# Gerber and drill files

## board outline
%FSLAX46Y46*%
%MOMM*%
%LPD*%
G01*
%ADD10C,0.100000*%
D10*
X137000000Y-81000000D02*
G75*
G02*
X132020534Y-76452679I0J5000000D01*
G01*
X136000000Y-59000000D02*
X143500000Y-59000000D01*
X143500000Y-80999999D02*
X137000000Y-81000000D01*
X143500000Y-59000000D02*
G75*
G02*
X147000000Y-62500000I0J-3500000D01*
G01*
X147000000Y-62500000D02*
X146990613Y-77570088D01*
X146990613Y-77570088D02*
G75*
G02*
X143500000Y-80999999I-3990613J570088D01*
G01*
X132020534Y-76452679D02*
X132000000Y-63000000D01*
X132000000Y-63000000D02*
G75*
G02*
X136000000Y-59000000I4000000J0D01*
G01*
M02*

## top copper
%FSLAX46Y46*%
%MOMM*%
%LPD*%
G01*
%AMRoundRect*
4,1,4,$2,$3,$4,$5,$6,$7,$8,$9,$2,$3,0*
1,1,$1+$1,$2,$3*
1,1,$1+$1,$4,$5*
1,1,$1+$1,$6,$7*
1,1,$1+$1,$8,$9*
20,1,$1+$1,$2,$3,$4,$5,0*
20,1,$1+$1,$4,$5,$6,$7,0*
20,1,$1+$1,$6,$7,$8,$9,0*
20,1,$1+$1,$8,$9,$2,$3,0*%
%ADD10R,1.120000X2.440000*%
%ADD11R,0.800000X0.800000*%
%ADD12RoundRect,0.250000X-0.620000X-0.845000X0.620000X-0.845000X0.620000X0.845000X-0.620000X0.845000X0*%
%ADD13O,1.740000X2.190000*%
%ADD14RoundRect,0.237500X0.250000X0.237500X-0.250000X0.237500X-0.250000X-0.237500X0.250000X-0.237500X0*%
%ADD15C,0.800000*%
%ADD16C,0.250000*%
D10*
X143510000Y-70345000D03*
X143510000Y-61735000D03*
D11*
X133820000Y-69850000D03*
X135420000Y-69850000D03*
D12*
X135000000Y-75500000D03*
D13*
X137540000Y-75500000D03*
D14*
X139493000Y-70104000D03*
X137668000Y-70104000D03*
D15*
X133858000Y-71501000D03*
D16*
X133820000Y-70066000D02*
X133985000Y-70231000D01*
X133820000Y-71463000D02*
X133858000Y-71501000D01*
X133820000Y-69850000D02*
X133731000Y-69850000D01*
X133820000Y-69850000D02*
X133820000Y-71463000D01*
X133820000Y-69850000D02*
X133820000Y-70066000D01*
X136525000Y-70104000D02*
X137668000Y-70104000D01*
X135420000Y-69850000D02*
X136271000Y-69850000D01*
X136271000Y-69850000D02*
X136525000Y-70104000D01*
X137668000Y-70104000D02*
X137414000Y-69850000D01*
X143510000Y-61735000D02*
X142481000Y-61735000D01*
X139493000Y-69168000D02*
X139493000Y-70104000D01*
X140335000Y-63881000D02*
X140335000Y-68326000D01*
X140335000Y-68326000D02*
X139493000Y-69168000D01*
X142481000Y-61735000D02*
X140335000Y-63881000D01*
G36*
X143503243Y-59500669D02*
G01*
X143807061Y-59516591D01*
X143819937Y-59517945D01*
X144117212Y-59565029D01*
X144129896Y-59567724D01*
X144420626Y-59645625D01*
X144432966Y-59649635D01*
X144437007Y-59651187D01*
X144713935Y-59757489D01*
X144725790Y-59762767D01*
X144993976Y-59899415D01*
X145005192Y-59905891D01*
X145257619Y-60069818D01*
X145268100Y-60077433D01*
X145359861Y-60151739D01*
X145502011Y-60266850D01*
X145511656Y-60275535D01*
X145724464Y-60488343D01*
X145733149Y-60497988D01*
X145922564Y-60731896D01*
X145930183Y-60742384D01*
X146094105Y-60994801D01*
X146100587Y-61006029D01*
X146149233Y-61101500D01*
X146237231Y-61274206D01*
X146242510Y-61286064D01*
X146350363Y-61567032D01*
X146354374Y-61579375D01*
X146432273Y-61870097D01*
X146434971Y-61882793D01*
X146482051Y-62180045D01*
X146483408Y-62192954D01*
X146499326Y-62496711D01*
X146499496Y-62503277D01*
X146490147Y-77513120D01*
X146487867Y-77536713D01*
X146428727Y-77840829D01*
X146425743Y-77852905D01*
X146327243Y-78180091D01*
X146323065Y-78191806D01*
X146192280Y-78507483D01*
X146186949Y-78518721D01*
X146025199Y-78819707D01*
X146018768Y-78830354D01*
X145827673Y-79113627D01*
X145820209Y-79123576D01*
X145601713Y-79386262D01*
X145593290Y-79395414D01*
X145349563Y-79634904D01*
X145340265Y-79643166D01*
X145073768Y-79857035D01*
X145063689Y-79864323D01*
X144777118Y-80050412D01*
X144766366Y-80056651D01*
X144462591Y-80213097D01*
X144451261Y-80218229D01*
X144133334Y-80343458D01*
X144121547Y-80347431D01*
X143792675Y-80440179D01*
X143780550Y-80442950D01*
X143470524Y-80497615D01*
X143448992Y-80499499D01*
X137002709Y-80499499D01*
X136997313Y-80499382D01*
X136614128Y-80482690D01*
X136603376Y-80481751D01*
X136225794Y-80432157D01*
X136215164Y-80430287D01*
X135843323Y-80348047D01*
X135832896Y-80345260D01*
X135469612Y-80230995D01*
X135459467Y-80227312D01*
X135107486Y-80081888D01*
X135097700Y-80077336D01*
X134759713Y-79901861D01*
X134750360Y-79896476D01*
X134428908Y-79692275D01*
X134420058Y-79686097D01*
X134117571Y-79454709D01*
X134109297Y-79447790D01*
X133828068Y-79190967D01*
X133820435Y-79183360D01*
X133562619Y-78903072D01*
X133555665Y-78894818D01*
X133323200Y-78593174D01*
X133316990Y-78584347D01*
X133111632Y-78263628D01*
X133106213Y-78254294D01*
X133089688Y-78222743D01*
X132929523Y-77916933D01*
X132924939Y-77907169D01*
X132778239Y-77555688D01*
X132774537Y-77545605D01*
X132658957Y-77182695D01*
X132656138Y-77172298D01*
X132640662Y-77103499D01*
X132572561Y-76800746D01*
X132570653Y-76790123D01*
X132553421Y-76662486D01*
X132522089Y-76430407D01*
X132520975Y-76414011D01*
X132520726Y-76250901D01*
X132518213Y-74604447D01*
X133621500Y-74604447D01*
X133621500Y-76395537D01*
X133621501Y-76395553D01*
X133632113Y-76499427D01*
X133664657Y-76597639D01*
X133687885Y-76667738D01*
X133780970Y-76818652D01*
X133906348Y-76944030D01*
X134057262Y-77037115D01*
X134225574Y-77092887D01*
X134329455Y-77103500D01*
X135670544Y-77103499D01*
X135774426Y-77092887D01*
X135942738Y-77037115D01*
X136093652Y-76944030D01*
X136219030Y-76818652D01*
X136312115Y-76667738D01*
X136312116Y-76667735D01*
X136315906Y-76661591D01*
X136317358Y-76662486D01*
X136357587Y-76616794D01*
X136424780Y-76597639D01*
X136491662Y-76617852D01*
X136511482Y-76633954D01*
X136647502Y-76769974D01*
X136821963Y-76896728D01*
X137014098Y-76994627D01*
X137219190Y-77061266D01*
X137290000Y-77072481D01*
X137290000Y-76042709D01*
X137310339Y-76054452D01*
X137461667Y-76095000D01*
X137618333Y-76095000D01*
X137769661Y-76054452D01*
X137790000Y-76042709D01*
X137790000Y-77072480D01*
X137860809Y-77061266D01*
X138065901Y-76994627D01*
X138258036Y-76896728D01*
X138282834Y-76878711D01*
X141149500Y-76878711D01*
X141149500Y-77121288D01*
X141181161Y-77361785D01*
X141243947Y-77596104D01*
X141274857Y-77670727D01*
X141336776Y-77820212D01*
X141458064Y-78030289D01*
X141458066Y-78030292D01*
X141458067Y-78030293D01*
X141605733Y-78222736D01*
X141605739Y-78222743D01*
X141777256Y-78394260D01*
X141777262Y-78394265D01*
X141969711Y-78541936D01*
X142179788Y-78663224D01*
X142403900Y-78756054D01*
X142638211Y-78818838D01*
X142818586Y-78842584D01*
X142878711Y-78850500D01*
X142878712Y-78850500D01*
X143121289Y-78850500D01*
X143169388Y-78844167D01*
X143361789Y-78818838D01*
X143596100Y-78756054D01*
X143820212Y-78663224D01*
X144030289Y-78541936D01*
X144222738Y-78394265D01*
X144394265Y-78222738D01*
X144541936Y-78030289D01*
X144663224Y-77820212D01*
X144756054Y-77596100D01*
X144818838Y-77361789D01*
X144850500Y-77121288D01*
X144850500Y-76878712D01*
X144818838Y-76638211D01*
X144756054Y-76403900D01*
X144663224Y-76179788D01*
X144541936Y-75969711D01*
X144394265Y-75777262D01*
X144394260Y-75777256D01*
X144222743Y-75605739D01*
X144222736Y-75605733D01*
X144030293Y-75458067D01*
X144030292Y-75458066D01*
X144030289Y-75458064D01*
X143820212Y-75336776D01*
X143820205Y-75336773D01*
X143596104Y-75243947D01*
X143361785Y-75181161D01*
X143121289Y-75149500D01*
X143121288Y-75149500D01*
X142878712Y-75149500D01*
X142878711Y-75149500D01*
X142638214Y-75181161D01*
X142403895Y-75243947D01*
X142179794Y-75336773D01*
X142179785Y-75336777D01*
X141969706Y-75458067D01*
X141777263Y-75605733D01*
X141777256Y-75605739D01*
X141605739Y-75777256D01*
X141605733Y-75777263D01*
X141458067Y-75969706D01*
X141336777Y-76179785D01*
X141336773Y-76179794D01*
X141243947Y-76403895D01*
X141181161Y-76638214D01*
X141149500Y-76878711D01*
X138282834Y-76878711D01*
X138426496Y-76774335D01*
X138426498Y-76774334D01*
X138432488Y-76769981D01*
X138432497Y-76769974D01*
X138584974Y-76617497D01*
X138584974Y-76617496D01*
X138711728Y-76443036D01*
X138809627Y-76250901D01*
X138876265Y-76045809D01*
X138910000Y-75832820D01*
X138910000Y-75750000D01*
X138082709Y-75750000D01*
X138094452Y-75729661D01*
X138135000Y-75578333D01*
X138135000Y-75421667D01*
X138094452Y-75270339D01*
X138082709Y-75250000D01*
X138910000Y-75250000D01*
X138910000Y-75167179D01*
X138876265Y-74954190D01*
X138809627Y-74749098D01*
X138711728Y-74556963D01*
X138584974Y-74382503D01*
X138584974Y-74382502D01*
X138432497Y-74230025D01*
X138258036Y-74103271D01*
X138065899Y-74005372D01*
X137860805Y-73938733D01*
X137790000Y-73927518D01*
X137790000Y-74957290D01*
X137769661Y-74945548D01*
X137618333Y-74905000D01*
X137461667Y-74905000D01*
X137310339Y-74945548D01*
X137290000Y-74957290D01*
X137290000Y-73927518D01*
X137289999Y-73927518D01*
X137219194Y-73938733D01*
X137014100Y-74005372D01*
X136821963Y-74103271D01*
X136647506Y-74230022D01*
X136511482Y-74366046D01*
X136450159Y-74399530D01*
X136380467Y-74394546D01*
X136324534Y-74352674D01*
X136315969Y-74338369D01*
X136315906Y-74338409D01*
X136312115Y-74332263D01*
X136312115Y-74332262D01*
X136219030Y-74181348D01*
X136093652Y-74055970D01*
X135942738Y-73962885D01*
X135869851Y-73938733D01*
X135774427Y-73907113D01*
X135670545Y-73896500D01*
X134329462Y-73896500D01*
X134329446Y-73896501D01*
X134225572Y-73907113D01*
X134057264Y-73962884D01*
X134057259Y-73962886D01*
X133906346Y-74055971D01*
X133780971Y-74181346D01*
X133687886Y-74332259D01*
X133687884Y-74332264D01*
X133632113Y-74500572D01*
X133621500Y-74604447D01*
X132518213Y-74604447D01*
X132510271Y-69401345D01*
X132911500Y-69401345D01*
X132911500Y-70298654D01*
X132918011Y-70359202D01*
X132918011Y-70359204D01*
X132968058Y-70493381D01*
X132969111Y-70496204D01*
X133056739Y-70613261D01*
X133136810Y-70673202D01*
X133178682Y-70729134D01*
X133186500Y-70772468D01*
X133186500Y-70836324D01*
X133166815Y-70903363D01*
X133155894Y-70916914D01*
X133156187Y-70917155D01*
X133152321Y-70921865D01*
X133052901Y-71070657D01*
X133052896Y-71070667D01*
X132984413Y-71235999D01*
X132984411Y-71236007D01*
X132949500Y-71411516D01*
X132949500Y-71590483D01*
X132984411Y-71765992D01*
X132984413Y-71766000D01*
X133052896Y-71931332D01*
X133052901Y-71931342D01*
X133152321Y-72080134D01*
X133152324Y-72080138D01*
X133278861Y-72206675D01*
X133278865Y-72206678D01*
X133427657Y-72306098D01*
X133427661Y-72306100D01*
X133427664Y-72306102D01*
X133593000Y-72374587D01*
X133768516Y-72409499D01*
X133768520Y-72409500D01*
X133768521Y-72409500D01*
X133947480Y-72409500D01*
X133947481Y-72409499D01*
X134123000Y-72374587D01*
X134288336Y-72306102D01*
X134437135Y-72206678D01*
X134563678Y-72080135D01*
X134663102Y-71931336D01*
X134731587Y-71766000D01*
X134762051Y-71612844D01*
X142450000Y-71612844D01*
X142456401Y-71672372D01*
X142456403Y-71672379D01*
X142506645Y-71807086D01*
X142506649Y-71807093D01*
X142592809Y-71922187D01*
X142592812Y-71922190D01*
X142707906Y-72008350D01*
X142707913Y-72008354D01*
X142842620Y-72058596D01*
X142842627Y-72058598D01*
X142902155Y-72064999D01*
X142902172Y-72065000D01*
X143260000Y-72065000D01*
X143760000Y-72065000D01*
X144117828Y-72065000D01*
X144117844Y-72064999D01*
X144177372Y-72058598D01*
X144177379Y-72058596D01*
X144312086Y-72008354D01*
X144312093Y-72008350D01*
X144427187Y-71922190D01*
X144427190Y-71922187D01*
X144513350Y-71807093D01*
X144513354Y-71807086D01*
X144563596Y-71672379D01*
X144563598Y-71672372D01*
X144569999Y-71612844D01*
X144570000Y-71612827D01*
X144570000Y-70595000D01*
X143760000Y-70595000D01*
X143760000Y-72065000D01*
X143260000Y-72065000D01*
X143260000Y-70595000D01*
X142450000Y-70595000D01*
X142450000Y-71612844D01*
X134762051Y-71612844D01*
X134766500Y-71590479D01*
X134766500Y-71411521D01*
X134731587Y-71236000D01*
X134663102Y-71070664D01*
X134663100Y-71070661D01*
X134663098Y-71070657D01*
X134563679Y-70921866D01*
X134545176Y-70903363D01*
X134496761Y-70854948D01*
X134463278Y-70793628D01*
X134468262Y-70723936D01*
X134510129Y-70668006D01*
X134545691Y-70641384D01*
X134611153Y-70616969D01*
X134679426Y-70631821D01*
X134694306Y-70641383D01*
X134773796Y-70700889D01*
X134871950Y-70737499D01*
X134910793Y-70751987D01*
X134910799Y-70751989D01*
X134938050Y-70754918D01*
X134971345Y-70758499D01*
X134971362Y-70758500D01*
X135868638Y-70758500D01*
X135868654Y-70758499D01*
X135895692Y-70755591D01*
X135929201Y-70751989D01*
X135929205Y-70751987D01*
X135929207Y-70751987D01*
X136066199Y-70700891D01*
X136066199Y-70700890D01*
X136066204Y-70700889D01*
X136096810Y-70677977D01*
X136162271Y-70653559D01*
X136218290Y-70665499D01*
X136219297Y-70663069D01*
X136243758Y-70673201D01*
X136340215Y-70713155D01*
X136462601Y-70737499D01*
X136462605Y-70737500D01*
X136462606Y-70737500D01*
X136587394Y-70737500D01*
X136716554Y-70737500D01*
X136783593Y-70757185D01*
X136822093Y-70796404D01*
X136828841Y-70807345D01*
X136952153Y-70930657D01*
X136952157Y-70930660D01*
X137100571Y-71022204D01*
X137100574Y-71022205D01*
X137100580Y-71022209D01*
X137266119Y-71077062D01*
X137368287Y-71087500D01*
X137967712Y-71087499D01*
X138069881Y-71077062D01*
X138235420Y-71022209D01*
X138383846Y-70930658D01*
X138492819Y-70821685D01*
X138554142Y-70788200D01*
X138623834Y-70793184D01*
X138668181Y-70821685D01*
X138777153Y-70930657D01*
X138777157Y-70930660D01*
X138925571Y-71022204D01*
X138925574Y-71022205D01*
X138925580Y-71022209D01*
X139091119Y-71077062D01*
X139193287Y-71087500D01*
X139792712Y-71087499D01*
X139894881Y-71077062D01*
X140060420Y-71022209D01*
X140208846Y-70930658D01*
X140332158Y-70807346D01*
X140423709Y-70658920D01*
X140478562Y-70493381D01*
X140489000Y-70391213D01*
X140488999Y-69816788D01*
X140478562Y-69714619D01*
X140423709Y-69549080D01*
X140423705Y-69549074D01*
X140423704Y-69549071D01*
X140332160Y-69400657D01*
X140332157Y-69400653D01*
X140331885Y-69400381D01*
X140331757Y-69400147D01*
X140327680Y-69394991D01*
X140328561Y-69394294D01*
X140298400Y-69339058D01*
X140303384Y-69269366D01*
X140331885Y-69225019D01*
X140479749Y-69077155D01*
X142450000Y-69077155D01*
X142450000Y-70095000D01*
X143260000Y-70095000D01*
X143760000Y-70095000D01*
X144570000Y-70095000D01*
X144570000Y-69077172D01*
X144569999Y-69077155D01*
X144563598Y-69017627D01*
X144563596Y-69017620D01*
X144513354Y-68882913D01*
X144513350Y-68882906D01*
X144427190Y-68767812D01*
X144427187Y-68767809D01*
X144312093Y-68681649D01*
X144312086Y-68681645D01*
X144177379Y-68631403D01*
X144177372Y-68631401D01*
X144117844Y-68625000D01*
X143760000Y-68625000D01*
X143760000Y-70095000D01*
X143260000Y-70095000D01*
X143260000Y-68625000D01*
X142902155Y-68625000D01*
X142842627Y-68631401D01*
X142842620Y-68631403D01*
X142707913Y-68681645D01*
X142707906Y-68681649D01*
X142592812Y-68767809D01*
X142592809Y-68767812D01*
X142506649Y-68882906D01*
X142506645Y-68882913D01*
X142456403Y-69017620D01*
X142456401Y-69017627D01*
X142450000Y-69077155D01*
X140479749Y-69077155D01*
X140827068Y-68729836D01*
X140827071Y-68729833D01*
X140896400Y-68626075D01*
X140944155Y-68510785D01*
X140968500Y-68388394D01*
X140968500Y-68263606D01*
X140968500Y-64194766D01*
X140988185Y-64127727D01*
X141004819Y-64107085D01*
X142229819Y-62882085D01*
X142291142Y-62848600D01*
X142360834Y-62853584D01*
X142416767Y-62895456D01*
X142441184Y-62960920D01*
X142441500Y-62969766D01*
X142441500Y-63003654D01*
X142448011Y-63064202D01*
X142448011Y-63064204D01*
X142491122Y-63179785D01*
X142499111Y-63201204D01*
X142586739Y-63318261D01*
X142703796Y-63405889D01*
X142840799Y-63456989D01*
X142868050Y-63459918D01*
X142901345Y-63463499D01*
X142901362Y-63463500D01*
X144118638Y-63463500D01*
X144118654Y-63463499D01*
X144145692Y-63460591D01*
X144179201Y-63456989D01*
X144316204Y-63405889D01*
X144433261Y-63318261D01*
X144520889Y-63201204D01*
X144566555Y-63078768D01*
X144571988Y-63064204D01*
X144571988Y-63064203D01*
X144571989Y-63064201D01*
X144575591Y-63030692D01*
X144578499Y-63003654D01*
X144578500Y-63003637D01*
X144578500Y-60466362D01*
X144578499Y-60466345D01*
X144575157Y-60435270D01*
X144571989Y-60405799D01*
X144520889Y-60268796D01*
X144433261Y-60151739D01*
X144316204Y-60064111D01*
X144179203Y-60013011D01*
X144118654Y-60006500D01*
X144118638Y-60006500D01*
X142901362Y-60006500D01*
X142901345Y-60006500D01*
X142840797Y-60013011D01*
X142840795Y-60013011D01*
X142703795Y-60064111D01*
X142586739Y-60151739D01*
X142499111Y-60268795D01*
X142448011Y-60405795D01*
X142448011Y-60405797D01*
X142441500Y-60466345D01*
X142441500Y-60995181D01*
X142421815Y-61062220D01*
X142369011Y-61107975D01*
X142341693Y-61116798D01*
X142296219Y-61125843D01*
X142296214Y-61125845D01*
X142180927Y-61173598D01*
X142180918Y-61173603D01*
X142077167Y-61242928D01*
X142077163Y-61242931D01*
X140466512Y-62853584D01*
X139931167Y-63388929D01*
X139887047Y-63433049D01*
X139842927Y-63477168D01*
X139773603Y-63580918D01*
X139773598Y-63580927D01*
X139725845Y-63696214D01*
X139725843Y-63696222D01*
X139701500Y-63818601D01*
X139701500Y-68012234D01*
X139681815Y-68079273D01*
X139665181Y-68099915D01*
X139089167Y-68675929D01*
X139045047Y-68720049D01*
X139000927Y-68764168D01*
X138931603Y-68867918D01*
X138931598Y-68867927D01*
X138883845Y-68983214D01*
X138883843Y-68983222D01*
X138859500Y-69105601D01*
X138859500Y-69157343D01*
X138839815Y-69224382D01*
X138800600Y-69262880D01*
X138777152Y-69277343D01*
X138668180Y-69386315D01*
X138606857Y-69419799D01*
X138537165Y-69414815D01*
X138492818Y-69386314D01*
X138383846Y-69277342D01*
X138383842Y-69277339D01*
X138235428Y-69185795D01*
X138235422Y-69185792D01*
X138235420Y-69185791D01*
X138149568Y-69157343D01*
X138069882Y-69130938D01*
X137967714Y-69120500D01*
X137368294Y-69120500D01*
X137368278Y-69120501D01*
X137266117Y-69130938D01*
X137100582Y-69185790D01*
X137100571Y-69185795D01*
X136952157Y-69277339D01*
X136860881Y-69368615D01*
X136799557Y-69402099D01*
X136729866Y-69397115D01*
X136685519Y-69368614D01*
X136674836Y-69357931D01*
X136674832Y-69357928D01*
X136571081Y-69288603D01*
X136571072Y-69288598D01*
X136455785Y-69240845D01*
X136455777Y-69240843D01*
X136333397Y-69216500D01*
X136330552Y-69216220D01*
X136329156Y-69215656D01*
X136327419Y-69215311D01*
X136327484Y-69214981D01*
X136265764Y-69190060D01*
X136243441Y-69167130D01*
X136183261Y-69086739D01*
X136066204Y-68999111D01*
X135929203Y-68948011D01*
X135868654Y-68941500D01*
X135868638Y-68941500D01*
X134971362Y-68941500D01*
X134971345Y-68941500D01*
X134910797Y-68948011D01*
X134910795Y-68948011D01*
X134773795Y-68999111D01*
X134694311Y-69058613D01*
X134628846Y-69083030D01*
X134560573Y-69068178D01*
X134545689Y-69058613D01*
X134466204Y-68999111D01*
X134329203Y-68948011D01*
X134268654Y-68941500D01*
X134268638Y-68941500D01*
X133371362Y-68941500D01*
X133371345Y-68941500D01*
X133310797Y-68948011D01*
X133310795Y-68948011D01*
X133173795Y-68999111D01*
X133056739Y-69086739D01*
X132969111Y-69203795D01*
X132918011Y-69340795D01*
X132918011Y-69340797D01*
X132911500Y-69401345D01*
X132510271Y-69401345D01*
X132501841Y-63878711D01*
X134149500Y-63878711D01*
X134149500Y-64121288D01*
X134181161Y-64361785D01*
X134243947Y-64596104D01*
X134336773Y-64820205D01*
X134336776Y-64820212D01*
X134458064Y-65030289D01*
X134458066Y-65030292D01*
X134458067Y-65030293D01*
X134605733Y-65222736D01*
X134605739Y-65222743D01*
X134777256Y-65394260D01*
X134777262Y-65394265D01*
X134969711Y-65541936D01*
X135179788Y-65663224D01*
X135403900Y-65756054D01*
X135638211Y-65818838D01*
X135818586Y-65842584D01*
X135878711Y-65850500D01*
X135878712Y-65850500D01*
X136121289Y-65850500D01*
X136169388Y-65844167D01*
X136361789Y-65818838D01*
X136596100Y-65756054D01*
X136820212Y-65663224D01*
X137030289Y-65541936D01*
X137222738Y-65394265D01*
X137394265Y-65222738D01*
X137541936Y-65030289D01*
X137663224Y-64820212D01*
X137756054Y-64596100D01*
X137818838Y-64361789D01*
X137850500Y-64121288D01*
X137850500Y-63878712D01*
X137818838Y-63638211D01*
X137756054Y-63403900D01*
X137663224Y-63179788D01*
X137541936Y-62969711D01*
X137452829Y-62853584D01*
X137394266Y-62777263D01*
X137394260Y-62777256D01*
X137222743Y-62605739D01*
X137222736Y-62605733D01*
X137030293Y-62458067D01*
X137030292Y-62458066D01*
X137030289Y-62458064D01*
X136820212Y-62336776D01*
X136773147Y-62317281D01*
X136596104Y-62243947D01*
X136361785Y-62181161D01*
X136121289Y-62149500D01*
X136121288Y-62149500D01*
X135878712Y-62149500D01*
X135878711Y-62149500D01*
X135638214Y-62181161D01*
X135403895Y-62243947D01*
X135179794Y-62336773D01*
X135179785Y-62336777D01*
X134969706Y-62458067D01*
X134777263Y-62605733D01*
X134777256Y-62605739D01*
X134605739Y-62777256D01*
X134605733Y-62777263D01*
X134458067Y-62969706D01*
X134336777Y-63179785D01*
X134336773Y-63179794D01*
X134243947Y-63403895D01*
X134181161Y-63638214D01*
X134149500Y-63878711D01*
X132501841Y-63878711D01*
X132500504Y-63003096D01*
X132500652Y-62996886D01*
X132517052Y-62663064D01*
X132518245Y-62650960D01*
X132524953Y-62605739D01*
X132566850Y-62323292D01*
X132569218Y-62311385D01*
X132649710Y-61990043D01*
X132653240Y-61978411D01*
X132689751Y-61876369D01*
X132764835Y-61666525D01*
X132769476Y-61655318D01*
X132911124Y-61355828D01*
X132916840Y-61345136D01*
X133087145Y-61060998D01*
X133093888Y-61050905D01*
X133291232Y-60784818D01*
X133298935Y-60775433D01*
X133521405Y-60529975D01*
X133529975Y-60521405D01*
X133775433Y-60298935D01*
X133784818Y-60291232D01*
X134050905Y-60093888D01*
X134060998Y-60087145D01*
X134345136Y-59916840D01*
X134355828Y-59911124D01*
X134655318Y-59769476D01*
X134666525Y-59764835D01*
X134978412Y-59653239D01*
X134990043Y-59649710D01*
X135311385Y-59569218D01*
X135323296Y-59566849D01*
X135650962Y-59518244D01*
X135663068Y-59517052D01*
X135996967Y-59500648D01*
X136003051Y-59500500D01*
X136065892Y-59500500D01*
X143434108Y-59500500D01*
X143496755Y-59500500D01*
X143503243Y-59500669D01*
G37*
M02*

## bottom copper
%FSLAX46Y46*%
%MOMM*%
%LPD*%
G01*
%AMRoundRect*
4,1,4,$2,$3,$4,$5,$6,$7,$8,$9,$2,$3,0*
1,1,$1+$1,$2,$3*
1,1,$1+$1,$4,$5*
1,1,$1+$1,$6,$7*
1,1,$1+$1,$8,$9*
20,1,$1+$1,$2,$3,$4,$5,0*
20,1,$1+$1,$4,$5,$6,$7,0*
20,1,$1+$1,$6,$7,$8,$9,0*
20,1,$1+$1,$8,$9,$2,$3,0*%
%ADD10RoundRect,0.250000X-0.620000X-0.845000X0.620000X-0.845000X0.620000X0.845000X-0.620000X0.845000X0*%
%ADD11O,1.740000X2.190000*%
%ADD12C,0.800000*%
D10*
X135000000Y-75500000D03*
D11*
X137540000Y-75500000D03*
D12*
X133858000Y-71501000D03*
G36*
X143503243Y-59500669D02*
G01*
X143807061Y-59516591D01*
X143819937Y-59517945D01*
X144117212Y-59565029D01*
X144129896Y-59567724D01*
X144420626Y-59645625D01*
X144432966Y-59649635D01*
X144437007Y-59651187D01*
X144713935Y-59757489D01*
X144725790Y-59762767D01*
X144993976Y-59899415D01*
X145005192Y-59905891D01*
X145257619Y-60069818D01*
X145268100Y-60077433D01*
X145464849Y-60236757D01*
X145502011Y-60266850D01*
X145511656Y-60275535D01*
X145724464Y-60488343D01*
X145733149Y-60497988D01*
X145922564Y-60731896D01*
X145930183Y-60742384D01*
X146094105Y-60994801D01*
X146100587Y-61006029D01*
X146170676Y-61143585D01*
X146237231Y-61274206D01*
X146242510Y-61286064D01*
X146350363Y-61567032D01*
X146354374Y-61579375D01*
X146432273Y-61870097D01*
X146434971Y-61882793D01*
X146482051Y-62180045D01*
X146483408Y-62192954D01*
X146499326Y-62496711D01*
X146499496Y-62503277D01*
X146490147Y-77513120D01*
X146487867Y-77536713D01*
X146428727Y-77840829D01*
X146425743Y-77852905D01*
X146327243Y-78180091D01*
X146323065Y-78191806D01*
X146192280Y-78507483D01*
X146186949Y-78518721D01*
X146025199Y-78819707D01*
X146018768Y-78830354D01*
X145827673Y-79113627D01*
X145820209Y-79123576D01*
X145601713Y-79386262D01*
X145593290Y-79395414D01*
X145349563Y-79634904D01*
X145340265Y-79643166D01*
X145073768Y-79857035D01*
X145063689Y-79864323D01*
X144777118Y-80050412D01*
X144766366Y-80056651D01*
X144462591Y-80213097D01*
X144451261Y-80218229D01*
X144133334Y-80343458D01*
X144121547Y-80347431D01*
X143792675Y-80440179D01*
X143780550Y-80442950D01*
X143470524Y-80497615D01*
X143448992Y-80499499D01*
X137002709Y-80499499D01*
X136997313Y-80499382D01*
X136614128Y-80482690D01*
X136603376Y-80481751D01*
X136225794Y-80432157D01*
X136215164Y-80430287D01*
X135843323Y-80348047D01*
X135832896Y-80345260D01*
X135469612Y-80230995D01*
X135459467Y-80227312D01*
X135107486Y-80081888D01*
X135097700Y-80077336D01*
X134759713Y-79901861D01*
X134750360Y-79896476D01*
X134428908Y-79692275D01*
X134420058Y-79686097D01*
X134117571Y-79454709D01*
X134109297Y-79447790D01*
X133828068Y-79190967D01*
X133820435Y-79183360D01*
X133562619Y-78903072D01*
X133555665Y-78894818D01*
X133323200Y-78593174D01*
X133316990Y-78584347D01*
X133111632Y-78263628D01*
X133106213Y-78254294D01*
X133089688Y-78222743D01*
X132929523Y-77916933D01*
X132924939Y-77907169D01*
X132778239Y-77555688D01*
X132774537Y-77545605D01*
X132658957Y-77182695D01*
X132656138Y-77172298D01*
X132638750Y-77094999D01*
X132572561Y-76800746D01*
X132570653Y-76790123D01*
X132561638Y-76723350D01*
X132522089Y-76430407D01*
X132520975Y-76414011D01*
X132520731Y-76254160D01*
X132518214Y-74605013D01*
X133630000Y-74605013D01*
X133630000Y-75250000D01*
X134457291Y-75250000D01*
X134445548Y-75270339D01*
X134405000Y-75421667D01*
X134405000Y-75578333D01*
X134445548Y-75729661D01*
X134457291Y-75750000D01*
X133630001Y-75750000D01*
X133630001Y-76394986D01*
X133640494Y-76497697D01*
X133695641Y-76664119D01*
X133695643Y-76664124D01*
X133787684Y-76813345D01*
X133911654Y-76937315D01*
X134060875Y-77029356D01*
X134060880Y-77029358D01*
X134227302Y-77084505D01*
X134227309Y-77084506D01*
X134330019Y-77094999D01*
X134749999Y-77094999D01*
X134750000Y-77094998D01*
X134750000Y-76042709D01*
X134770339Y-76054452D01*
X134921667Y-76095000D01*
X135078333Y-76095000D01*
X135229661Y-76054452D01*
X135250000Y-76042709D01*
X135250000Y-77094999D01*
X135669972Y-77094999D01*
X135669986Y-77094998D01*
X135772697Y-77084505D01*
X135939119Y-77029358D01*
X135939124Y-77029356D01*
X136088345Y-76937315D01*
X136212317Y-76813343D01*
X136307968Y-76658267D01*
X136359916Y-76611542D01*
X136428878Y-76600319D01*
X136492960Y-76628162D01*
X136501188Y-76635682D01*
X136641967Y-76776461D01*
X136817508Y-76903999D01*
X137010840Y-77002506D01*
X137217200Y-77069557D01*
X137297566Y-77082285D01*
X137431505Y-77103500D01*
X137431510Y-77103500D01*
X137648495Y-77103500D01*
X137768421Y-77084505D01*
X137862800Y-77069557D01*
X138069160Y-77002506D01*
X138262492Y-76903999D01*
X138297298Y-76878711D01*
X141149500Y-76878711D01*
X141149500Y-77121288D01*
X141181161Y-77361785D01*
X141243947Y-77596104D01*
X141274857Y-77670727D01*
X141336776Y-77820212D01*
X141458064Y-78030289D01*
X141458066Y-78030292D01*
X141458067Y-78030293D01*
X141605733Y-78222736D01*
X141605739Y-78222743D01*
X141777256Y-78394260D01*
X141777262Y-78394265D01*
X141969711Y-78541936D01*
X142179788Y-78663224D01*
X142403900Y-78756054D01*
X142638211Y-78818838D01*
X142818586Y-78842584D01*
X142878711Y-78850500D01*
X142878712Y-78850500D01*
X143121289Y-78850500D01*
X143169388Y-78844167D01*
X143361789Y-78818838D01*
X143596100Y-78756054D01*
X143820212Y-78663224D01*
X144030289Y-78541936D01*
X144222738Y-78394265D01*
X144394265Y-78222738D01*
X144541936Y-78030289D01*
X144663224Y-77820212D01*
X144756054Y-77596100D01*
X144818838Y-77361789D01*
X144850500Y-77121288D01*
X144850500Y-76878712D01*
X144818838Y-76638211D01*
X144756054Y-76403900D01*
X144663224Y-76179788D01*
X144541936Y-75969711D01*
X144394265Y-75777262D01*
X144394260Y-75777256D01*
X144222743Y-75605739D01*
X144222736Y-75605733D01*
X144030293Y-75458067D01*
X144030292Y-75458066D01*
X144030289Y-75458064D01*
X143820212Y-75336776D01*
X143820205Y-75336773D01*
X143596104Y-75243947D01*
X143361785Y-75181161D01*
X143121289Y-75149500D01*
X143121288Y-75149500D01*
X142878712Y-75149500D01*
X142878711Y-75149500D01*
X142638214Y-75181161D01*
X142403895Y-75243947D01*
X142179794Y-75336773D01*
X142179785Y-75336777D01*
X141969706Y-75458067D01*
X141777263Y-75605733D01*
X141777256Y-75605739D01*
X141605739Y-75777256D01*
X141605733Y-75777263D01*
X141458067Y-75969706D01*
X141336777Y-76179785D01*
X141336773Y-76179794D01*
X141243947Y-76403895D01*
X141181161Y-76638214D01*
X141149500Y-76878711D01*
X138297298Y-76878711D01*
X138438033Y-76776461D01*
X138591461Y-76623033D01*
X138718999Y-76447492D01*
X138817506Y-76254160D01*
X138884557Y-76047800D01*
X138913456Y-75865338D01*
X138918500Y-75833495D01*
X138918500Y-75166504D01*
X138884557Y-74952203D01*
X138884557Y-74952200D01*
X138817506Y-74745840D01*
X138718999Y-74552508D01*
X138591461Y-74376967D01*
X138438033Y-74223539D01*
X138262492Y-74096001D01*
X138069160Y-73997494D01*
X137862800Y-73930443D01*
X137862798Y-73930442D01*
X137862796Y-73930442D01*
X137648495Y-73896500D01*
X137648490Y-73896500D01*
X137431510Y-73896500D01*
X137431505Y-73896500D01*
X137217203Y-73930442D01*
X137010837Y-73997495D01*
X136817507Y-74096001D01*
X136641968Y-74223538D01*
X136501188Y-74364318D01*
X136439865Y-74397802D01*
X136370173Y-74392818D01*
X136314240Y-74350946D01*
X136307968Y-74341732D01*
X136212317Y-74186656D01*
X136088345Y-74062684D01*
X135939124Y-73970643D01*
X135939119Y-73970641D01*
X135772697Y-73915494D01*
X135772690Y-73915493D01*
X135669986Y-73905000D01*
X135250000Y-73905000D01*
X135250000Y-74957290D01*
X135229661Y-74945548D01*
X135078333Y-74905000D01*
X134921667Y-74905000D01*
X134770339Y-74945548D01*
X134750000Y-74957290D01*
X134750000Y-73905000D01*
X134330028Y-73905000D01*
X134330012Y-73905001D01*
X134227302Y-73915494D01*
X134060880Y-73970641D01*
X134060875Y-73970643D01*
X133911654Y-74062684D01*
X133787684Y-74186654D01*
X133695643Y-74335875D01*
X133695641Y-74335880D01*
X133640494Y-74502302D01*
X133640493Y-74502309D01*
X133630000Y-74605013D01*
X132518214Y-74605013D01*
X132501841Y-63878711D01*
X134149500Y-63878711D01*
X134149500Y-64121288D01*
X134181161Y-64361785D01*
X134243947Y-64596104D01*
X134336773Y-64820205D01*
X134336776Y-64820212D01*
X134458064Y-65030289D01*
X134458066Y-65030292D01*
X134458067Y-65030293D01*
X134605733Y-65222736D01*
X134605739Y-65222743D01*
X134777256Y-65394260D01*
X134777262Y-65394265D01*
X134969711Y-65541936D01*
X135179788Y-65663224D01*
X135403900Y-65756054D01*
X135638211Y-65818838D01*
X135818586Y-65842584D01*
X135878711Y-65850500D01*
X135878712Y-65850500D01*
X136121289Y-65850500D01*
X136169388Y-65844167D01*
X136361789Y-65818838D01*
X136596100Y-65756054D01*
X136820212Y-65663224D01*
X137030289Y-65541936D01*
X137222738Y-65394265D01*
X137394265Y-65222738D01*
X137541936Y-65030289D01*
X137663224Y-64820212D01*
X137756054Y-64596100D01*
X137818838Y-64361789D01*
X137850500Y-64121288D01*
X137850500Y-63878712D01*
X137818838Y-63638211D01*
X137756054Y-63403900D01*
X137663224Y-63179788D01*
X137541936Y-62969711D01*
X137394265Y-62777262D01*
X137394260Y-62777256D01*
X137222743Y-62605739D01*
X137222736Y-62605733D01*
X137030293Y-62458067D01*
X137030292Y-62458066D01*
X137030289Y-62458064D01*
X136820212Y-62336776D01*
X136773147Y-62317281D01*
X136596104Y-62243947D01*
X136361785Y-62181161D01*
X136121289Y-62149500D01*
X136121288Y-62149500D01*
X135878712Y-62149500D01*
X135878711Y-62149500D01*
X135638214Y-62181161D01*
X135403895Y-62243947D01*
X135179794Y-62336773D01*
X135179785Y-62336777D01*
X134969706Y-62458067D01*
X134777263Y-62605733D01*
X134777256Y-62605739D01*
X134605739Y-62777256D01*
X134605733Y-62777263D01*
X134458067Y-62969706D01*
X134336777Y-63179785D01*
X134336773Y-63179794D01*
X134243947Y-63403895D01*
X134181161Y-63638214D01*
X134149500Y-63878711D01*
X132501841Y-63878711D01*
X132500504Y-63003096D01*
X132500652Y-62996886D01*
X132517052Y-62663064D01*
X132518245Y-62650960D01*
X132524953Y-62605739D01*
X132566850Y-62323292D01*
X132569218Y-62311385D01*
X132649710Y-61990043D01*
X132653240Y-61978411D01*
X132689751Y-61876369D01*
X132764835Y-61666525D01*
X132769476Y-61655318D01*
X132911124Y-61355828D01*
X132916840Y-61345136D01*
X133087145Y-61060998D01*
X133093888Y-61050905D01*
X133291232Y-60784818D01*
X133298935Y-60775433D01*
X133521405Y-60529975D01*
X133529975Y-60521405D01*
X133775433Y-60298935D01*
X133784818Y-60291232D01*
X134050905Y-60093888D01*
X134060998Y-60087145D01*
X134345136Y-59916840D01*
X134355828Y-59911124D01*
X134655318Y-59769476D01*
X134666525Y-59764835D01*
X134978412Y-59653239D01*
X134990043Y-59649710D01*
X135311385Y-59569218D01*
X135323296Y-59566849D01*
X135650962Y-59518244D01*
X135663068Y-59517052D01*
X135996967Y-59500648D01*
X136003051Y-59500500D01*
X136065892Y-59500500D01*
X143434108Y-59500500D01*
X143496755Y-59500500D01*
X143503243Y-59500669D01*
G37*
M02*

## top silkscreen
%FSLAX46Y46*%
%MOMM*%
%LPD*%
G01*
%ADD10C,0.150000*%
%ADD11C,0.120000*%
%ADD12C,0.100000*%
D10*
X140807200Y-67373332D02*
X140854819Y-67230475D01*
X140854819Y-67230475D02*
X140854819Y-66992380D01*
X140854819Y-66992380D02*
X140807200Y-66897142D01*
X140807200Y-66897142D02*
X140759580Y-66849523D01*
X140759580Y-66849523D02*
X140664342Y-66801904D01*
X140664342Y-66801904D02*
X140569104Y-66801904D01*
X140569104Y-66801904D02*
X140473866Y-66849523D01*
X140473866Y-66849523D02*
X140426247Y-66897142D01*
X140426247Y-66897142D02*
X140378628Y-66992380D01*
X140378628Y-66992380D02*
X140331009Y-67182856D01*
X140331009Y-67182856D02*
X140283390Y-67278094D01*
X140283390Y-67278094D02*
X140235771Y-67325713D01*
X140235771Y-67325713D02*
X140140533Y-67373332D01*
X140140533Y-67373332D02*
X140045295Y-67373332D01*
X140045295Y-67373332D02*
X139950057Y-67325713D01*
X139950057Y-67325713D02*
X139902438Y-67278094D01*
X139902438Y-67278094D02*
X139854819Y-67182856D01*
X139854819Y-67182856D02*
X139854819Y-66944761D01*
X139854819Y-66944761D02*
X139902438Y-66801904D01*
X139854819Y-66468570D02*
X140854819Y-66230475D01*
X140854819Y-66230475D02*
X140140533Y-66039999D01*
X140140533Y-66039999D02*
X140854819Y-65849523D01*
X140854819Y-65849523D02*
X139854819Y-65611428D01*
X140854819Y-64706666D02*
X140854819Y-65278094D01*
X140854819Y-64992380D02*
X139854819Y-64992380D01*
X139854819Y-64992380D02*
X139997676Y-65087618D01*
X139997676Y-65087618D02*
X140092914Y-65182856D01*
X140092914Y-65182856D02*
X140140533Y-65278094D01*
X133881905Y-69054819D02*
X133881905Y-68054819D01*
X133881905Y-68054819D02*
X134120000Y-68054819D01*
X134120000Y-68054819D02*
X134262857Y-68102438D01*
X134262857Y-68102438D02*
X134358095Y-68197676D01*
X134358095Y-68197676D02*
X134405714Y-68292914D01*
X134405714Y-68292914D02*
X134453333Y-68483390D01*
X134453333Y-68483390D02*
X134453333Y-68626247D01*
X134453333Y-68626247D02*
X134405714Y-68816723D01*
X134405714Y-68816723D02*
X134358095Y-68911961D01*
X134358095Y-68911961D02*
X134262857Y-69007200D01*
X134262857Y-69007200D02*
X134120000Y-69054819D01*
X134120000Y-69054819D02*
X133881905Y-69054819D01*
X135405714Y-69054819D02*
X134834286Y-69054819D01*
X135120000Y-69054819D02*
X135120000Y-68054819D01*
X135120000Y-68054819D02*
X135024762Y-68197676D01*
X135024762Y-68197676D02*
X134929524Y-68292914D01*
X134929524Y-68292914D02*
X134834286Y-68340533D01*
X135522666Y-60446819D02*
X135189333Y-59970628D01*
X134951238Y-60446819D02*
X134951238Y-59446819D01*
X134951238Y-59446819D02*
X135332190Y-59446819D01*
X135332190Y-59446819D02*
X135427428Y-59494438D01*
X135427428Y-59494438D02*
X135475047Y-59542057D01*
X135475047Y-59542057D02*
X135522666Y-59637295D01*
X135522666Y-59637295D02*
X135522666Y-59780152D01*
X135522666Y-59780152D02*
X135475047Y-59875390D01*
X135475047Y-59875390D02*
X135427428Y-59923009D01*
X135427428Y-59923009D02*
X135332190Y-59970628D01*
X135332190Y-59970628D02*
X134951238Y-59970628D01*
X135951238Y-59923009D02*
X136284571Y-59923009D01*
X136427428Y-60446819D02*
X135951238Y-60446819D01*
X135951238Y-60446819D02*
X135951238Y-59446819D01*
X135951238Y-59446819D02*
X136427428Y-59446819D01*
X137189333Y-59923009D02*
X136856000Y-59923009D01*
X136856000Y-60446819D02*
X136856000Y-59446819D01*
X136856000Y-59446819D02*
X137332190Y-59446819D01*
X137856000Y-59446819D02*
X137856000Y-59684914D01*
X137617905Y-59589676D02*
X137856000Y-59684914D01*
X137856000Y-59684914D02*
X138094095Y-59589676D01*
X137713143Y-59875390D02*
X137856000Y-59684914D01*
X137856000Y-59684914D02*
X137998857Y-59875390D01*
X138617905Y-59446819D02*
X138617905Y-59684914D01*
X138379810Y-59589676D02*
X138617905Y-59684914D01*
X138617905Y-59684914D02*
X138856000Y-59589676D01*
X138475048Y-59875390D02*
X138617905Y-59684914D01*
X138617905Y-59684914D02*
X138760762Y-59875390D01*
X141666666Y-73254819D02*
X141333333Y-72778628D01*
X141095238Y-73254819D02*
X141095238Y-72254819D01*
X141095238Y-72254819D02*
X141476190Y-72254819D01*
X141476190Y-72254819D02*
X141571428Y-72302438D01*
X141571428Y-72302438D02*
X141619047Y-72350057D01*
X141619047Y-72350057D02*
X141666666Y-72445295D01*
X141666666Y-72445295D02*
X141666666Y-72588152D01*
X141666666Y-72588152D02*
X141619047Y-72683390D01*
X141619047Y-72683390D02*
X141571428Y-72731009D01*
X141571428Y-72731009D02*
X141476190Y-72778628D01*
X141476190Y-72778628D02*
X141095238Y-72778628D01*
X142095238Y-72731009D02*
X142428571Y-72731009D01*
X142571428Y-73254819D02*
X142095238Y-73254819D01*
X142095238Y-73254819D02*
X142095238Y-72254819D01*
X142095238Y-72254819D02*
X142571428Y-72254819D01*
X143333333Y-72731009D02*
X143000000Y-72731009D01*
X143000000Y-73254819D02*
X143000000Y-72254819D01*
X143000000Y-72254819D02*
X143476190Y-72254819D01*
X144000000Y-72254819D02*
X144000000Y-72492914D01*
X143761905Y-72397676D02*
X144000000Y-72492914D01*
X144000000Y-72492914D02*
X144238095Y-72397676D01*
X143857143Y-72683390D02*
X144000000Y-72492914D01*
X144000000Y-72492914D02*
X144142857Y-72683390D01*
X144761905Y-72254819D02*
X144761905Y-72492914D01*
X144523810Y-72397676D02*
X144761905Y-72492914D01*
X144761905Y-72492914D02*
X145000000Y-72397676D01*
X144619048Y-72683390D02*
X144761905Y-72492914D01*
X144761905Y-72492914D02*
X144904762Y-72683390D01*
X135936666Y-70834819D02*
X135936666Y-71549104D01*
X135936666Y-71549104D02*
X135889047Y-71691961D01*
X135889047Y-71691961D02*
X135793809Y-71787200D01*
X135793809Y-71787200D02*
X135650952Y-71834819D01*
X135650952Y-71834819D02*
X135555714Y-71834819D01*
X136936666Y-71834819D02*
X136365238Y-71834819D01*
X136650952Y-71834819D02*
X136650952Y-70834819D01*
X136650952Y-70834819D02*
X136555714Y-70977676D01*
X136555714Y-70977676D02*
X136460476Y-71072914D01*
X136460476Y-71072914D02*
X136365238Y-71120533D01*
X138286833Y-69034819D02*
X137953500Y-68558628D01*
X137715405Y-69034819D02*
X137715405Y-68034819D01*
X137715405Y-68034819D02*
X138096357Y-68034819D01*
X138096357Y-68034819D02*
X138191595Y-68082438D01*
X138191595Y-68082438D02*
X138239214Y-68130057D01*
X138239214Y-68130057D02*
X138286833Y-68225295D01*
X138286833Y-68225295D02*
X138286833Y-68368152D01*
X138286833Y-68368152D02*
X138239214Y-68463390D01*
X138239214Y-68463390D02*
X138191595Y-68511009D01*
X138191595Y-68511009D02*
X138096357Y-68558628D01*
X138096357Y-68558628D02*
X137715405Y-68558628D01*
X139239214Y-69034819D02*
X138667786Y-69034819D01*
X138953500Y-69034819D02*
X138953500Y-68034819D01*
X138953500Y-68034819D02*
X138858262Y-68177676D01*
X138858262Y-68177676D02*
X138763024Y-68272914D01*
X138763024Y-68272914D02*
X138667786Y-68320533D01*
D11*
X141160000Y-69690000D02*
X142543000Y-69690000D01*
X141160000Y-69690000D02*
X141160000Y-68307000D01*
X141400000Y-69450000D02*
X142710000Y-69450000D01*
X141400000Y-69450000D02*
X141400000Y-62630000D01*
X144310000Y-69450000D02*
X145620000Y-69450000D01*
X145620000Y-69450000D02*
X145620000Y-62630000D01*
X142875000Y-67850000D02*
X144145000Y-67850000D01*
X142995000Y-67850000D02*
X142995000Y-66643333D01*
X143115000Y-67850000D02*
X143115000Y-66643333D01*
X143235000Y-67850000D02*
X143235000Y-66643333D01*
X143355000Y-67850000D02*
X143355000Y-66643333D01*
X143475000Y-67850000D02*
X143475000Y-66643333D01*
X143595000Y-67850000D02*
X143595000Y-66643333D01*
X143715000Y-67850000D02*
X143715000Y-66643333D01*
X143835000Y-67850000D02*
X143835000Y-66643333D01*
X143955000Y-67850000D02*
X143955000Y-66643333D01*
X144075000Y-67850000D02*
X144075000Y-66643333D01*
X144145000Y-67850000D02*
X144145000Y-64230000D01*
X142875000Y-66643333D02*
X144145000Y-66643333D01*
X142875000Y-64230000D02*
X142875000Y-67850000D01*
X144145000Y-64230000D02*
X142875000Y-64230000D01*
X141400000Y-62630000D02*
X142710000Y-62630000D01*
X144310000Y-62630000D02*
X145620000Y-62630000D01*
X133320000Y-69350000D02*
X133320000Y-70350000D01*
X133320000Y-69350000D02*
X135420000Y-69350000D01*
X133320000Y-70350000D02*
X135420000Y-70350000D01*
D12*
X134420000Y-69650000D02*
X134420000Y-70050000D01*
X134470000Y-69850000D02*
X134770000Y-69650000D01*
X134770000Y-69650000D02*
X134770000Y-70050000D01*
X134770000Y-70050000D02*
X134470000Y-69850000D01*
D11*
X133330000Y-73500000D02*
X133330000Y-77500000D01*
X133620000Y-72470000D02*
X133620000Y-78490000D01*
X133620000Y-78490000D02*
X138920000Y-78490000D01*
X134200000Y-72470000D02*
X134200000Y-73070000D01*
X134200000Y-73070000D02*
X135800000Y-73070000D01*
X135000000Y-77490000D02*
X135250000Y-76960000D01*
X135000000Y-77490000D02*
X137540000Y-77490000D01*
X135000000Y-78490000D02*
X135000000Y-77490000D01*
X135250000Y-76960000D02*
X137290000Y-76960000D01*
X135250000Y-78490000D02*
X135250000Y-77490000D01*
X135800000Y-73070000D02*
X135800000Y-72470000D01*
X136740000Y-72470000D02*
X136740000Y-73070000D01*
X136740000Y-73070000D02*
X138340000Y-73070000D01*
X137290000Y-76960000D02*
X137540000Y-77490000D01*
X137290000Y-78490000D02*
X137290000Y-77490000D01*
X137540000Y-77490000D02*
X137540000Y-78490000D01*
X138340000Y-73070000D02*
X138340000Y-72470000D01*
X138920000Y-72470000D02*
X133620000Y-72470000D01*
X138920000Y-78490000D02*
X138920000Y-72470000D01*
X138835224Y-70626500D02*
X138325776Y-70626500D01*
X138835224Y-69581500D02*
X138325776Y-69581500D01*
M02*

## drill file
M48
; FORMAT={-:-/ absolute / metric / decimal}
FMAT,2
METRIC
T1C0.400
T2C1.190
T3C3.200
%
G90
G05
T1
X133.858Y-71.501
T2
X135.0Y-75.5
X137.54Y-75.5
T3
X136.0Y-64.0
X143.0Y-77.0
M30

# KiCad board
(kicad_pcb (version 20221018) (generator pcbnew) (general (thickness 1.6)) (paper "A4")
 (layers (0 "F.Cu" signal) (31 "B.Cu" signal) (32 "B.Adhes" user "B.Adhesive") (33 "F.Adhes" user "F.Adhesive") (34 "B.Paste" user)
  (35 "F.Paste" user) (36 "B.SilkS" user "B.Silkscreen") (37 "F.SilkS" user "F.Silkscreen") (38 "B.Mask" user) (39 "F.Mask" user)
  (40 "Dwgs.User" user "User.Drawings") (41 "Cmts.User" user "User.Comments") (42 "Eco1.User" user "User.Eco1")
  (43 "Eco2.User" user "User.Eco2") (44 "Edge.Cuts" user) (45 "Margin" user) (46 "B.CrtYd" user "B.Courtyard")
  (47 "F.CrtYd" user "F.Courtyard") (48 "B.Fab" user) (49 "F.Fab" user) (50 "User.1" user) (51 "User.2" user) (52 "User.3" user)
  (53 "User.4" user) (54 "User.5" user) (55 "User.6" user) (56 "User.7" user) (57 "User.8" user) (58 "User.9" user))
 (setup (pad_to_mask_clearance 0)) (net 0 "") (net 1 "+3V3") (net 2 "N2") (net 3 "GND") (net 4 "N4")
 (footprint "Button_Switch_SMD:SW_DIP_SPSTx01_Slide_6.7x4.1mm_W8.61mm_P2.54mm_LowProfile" (layer "F.Cu") (at 143.51 66.04 90)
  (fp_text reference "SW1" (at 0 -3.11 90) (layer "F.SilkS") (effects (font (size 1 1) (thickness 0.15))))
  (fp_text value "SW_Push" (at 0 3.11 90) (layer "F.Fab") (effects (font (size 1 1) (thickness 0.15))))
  (fp_line (start -3.65 -2.35) (end -3.65 -0.967) (stroke (width 0.12) (type solid)) (layer "F.SilkS"))
  (fp_line (start -3.65 -2.35) (end -2.267 -2.35) (stroke (width 0.12) (type solid)) (layer "F.SilkS"))
  (fp_line (start -3.41 -2.11) (end -3.41 -0.8) (stroke (width 0.12) (type solid)) (layer "F.SilkS"))
  (fp_line (start -3.41 -2.11) (end 3.41 -2.11) (stroke (width 0.12) (type solid)) (layer "F.SilkS"))
  (fp_line (start -3.41 0.8) (end -3.41 2.11) (stroke (width 0.12) (type solid)) (layer "F.SilkS"))
  (fp_line (start -3.41 2.11) (end 3.41 2.11) (stroke (width 0.12) (type solid)) (layer "F.SilkS"))
  (fp_line (start -1.81 -0.635) (end -1.81 0.635) (stroke (width 0.12) (type solid)) (layer "F.SilkS"))
  (fp_line (start -1.81 -0.515) (end -0.603333 -0.515) (stroke (width 0.12) (type solid)) (layer "F.SilkS"))
  (fp_line (start -1.81 -0.395) (end -0.603333 -0.395) (stroke (width 0.12) (type solid)) (layer "F.SilkS"))
  (fp_line (start -1.81 -0.275) (end -0.603333 -0.275) (stroke (width 0.12) (type solid)) (layer "F.SilkS"))
  (fp_line (start -1.81 -0.155) (end -0.603333 -0.155) (stroke (width 0.12) (type solid)) (layer "F.SilkS"))
  (fp_line (start -1.81 -0.035) (end -0.603333 -0.035) (stroke (width 0.12) (type solid)) (layer "F.SilkS"))
  (fp_line (start -1.81 0.085) (end -0.603333 0.085) (stroke (width 0.12) (type solid)) (layer "F.SilkS"))
  (fp_line (start -1.81 0.205) (end -0.603333 0.205) (stroke (width 0.12) (type solid)) (layer "F.SilkS"))
  (fp_line (start -1.81 0.325) (end -0.603333 0.325) (stroke (width 0.12) (type solid)) (layer "F.SilkS"))
  (fp_line (start -1.81 0.445) (end -0.603333 0.445) (stroke (width 0.12) (type solid)) (layer "F.SilkS"))
  (fp_line (start -1.81 0.565) (end -0.603333 0.565) (stroke (width 0.12) (type solid)) (layer "F.SilkS"))
  (fp_line (start -1.81 0.635) (end 1.81 0.635) (stroke (width 0.12) (type solid)) (layer "F.SilkS"))
  (fp_line (start -0.603333 -0.635) (end -0.603333 0.635) (stroke (width 0.12) (type solid)) (layer "F.SilkS"))
  (fp_line (start 1.81 -0.635) (end -1.81 -0.635) (stroke (width 0.12) (type solid)) (layer "F.SilkS"))
  (fp_line (start 1.81 0.635) (end 1.81 -0.635) (stroke (width 0.12) (type solid)) (layer "F.SilkS"))
  (fp_line (start 3.41 -2.11) (end 3.41 -0.8) (stroke (width 0.12) (type solid)) (layer "F.SilkS"))
  (fp_line (start 3.41 0.8) (end 3.41 2.11) (stroke (width 0.12) (type solid)) (layer "F.SilkS"))
  (pad "1" smd rect (at -4.305 0 90) (size 2.44 1.12) (layers "F.Cu" "F.Paste" "F.Mask") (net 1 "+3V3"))
  (pad "2" smd rect (at 4.305 0 90) (size 2.44 1.12) (layers "F.Cu" "F.Paste" "F.Mask") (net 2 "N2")))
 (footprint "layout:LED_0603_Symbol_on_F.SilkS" (layer "F.Cu") (at 134.62 69.85)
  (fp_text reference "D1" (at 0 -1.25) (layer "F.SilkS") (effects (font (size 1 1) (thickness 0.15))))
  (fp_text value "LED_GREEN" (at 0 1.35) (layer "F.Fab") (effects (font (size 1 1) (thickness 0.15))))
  (fp_line (start -1.3 -0.5) (end -1.3 0.5) (stroke (width 0.12) (type solid)) (layer "F.SilkS"))
  (fp_line (start -1.3 -0.5) (end 0.8 -0.5) (stroke (width 0.12) (type solid)) (layer "F.SilkS"))
  (fp_line (start -1.3 0.5) (end 0.8 0.5) (stroke (width 0.12) (type solid)) (layer "F.SilkS"))
  (fp_line (start -0.2 -0.2) (end -0.2 0.2) (stroke (width 0.1) (type solid)) (layer "F.SilkS"))
  (fp_line (start -0.15 0) (end 0.15 -0.2) (stroke (width 0.1) (type solid)) (layer "F.SilkS"))
  (fp_line (start 0.15 -0.2) (end 0.15 0.2) (stroke (width 0.1) (type solid)) (layer "F.SilkS"))
  (fp_line (start 0.15 0.2) (end -0.15 0) (stroke (width 0.1) (type solid)) (layer "F.SilkS"))
  (pad "1" smd rect (at -0.8 0 180) (size 0.8 0.8) (layers "F.Cu" "F.Paste" "F.Mask") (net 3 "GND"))
  (pad "2" smd rect (at 0.8 0 180) (size 0.8 0.8) (layers "F.Cu" "F.Paste" "F.Mask") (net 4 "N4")))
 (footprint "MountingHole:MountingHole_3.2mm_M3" (layer "F.Cu") (at 136 64)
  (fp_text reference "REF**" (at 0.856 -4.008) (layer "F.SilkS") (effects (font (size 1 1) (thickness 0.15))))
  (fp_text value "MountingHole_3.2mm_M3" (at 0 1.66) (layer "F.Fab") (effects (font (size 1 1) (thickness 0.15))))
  (pad "" np_thru_hole circle (at 0 0) (size 3.2 3.2) (drill 3.2) (layers "*.Cu" "*.Mask")))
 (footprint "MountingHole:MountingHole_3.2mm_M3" (layer "F.Cu") (at 143 77)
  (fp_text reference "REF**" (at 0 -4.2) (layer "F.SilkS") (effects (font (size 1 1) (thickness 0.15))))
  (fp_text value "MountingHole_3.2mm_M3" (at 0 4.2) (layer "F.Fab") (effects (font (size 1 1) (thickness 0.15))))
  (pad "" np_thru_hole circle (at 0 0) (size 3.2 3.2) (drill 3.2) (layers "F&B.Cu" "*.Mask")))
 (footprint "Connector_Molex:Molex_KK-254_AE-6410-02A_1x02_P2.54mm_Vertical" (layer "F.Cu") (at 135 75.5)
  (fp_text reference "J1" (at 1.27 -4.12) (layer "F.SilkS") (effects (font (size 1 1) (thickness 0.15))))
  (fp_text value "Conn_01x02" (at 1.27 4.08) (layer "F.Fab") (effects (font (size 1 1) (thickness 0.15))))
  (fp_line (start -1.67 -2) (end -1.67 2) (stroke (width 0.12) (type solid)) (layer "F.SilkS"))
  (fp_line (start -1.38 -3.03) (end -1.38 2.99) (stroke (width 0.12) (type solid)) (layer "F.SilkS"))
  (fp_line (start -1.38 2.99) (end 3.92 2.99) (stroke (width 0.12) (type solid)) (layer "F.SilkS"))
  (fp_line (start -0.8 -3.03) (end -0.8 -2.43) (stroke (width 0.12) (type solid)) (layer "F.SilkS"))
  (fp_line (start -0.8 -2.43) (end 0.8 -2.43) (stroke (width 0.12) (type solid)) (layer "F.SilkS"))
  (fp_line (start 0 1.99) (end 0.25 1.46) (stroke (width 0.12) (type solid)) (layer "F.SilkS"))
  (fp_line (start 0 1.99) (end 2.54 1.99) (stroke (width 0.12) (type solid)) (layer "F.SilkS"))
  (fp_line (start 0 2.99) (end 0 1.99) (stroke (width 0.12) (type solid)) (layer "F.SilkS"))
  (fp_line (start 0.25 1.46) (end 2.29 1.46) (stroke (width 0.12) (type solid)) (layer "F.SilkS"))
  (fp_line (start 0.25 2.99) (end 0.25 1.99) (stroke (width 0.12) (type solid)) (layer "F.SilkS"))
  (fp_line (start 0.8 -2.43) (end 0.8 -3.03) (stroke (width 0.12) (type solid)) (layer "F.SilkS"))
  (fp_line (start 1.74 -3.03) (end 1.74 -2.43) (stroke (width 0.12) (type solid)) (layer "F.SilkS"))
  (fp_line (start 1.74 -2.43) (end 3.34 -2.43) (stroke (width 0.12) (type solid)) (layer "F.SilkS"))
  (fp_line (start 2.29 1.46) (end 2.54 1.99) (stroke (width 0.12) (type solid)) (layer "F.SilkS"))
  (fp_line (start 2.29 2.99) (end 2.29 1.99) (stroke (width 0.12) (type solid)) (layer "F.SilkS"))
  (fp_line (start 2.54 1.99) (end 2.54 2.99) (stroke (width 0.12) (type solid)) (layer "F.SilkS"))
  (fp_line (start 3.34 -2.43) (end 3.34 -3.03) (stroke (width 0.12) (type solid)) (layer "F.SilkS"))
  (fp_line (start 3.92 -3.03) (end -1.38 -3.03) (stroke (width 0.12) (type solid)) (layer "F.SilkS"))
  (fp_line (start 3.92 2.99) (end 3.92 -3.03) (stroke (width 0.12) (type solid)) (layer "F.SilkS"))
  (pad "1" thru_hole roundrect (at 0 0) (size 1.74 2.19) (drill 1.19) (layers "*.Cu" "*.Mask") (roundrect_rratio 0.143678) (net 3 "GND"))
  (pad "2" thru_hole oval (at 2.54 0) (size 1.74 2.19) (drill 1.19) (layers "*.Cu" "*.Mask") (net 1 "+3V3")))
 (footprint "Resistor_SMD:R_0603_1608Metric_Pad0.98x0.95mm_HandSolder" (layer "F.Cu") (at 138.5805 70.104 180)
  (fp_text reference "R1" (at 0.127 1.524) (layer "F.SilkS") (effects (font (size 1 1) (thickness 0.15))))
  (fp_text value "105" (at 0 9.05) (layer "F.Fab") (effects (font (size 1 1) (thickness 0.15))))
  (fp_line (start -0.254724 -0.5225) (end 0.254724 -0.5225) (stroke (width 0.12) (type solid)) (layer "F.SilkS"))
  (fp_line (start -0.254724 0.5225) (end 0.254724 0.5225) (stroke (width 0.12) (type solid)) (layer "F.SilkS"))
  (pad "1" smd roundrect (at -0.9125 0 180) (size 0.975 0.95) (layers "F.Cu" "F.Paste" "F.Mask") (roundrect_rratio 0.25) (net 2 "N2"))
  (pad "2" smd roundrect (at 0.9125 0 180) (size 0.975 0.95) (layers "F.Cu" "F.Paste" "F.Mask") (roundrect_rratio 0.25) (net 4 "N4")))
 (gr_arc (start 137 81) (mid 133.628309 79.692113) (end 132.020534 76.452679) (stroke (width 0.1) (type default)) (layer "Edge.Cuts"))
 (gr_line (start 136 59) (end 143.5 59) (stroke (width 0.1) (type default)) (layer "Edge.Cuts"))
 (gr_line (start 143.5 80.999999) (end 137 81) (stroke (width 0.1) (type default)) (layer "Edge.Cuts"))
 (gr_arc (start 143.5 59) (mid 145.974874 60.025126) (end 147 62.5) (stroke (width 0.1) (type default)) (layer "Edge.Cuts"))
 (gr_line (start 147 62.5) (end 146.990613 77.570088) (stroke (width 0.1) (type default)) (layer "Edge.Cuts"))
 (gr_arc (start 146.990613 77.570088) (mid 145.825327 79.875329) (end 143.5 80.999999) (stroke (width 0.1) (type default))
  (layer "Edge.Cuts"))
 (gr_line (start 132.020534 76.452679) (end 132 63) (stroke (width 0.1) (type default)) (layer "Edge.Cuts"))
 (gr_arc (start 132 63) (mid 133.171573 60.171573) (end 136 59) (stroke (width 0.1) (type default)) (layer "Edge.Cuts"))
 (segment (start 133.82 70.066) (end 133.985 70.231) (width 0.25) (layer "F.Cu") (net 3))
 (segment (start 133.82 71.463) (end 133.858 71.501) (width 0.25) (layer "F.Cu") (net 3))
 (segment (start 133.82 69.85) (end 133.731 69.85) (width 0.25) (layer "F.Cu") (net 3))
 (segment (start 133.82 69.85) (end 133.82 71.463) (width 0.25) (layer "F.Cu") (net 3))
 (segment (start 133.82 69.85) (end 133.82 70.066) (width 0.25) (layer "F.Cu") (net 3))
 (via (at 133.858 71.501) (size 0.8) (drill 0.4) (layers "F.Cu" "B.Cu") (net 3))
 (segment (start 136.525 70.104) (end 137.668 70.104) (width 0.25) (layer "F.Cu") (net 4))
 (segment (start 135.42 69.85) (end 136.271 69.85) (width 0.25) (layer "F.Cu") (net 4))
 (segment (start 136.271 69.85) (end 136.525 70.104) (width 0.25) (layer "F.Cu") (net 4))
 (segment (start 137.668 70.104) (end 137.414 69.85) (width 0.25) (layer "F.Cu") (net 4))
 (segment (start 143.51 61.735) (end 142.481 61.735) (width 0.25) (layer "F.Cu") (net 2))
 (segment (start 139.493 69.168) (end 139.493 70.104) (width 0.25) (layer "F.Cu") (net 2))
 (segment (start 140.335 63.881) (end 140.335 68.326) (width 0.25) (layer "F.Cu") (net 2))
 (segment (start 140.335 68.326) (end 139.493 69.168) (width 0.25) (layer "F.Cu") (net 2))
 (segment (start 142.481 61.735) (end 140.335 63.881) (width 0.25) (layer "F.Cu") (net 2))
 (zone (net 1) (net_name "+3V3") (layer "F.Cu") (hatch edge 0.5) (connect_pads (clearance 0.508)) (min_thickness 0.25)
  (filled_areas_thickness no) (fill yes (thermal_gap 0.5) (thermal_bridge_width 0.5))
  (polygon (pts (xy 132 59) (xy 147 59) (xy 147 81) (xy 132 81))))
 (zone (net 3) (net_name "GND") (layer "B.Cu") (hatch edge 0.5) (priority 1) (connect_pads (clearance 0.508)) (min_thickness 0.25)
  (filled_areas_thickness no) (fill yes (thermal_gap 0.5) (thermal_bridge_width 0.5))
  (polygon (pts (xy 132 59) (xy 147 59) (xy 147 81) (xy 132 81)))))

